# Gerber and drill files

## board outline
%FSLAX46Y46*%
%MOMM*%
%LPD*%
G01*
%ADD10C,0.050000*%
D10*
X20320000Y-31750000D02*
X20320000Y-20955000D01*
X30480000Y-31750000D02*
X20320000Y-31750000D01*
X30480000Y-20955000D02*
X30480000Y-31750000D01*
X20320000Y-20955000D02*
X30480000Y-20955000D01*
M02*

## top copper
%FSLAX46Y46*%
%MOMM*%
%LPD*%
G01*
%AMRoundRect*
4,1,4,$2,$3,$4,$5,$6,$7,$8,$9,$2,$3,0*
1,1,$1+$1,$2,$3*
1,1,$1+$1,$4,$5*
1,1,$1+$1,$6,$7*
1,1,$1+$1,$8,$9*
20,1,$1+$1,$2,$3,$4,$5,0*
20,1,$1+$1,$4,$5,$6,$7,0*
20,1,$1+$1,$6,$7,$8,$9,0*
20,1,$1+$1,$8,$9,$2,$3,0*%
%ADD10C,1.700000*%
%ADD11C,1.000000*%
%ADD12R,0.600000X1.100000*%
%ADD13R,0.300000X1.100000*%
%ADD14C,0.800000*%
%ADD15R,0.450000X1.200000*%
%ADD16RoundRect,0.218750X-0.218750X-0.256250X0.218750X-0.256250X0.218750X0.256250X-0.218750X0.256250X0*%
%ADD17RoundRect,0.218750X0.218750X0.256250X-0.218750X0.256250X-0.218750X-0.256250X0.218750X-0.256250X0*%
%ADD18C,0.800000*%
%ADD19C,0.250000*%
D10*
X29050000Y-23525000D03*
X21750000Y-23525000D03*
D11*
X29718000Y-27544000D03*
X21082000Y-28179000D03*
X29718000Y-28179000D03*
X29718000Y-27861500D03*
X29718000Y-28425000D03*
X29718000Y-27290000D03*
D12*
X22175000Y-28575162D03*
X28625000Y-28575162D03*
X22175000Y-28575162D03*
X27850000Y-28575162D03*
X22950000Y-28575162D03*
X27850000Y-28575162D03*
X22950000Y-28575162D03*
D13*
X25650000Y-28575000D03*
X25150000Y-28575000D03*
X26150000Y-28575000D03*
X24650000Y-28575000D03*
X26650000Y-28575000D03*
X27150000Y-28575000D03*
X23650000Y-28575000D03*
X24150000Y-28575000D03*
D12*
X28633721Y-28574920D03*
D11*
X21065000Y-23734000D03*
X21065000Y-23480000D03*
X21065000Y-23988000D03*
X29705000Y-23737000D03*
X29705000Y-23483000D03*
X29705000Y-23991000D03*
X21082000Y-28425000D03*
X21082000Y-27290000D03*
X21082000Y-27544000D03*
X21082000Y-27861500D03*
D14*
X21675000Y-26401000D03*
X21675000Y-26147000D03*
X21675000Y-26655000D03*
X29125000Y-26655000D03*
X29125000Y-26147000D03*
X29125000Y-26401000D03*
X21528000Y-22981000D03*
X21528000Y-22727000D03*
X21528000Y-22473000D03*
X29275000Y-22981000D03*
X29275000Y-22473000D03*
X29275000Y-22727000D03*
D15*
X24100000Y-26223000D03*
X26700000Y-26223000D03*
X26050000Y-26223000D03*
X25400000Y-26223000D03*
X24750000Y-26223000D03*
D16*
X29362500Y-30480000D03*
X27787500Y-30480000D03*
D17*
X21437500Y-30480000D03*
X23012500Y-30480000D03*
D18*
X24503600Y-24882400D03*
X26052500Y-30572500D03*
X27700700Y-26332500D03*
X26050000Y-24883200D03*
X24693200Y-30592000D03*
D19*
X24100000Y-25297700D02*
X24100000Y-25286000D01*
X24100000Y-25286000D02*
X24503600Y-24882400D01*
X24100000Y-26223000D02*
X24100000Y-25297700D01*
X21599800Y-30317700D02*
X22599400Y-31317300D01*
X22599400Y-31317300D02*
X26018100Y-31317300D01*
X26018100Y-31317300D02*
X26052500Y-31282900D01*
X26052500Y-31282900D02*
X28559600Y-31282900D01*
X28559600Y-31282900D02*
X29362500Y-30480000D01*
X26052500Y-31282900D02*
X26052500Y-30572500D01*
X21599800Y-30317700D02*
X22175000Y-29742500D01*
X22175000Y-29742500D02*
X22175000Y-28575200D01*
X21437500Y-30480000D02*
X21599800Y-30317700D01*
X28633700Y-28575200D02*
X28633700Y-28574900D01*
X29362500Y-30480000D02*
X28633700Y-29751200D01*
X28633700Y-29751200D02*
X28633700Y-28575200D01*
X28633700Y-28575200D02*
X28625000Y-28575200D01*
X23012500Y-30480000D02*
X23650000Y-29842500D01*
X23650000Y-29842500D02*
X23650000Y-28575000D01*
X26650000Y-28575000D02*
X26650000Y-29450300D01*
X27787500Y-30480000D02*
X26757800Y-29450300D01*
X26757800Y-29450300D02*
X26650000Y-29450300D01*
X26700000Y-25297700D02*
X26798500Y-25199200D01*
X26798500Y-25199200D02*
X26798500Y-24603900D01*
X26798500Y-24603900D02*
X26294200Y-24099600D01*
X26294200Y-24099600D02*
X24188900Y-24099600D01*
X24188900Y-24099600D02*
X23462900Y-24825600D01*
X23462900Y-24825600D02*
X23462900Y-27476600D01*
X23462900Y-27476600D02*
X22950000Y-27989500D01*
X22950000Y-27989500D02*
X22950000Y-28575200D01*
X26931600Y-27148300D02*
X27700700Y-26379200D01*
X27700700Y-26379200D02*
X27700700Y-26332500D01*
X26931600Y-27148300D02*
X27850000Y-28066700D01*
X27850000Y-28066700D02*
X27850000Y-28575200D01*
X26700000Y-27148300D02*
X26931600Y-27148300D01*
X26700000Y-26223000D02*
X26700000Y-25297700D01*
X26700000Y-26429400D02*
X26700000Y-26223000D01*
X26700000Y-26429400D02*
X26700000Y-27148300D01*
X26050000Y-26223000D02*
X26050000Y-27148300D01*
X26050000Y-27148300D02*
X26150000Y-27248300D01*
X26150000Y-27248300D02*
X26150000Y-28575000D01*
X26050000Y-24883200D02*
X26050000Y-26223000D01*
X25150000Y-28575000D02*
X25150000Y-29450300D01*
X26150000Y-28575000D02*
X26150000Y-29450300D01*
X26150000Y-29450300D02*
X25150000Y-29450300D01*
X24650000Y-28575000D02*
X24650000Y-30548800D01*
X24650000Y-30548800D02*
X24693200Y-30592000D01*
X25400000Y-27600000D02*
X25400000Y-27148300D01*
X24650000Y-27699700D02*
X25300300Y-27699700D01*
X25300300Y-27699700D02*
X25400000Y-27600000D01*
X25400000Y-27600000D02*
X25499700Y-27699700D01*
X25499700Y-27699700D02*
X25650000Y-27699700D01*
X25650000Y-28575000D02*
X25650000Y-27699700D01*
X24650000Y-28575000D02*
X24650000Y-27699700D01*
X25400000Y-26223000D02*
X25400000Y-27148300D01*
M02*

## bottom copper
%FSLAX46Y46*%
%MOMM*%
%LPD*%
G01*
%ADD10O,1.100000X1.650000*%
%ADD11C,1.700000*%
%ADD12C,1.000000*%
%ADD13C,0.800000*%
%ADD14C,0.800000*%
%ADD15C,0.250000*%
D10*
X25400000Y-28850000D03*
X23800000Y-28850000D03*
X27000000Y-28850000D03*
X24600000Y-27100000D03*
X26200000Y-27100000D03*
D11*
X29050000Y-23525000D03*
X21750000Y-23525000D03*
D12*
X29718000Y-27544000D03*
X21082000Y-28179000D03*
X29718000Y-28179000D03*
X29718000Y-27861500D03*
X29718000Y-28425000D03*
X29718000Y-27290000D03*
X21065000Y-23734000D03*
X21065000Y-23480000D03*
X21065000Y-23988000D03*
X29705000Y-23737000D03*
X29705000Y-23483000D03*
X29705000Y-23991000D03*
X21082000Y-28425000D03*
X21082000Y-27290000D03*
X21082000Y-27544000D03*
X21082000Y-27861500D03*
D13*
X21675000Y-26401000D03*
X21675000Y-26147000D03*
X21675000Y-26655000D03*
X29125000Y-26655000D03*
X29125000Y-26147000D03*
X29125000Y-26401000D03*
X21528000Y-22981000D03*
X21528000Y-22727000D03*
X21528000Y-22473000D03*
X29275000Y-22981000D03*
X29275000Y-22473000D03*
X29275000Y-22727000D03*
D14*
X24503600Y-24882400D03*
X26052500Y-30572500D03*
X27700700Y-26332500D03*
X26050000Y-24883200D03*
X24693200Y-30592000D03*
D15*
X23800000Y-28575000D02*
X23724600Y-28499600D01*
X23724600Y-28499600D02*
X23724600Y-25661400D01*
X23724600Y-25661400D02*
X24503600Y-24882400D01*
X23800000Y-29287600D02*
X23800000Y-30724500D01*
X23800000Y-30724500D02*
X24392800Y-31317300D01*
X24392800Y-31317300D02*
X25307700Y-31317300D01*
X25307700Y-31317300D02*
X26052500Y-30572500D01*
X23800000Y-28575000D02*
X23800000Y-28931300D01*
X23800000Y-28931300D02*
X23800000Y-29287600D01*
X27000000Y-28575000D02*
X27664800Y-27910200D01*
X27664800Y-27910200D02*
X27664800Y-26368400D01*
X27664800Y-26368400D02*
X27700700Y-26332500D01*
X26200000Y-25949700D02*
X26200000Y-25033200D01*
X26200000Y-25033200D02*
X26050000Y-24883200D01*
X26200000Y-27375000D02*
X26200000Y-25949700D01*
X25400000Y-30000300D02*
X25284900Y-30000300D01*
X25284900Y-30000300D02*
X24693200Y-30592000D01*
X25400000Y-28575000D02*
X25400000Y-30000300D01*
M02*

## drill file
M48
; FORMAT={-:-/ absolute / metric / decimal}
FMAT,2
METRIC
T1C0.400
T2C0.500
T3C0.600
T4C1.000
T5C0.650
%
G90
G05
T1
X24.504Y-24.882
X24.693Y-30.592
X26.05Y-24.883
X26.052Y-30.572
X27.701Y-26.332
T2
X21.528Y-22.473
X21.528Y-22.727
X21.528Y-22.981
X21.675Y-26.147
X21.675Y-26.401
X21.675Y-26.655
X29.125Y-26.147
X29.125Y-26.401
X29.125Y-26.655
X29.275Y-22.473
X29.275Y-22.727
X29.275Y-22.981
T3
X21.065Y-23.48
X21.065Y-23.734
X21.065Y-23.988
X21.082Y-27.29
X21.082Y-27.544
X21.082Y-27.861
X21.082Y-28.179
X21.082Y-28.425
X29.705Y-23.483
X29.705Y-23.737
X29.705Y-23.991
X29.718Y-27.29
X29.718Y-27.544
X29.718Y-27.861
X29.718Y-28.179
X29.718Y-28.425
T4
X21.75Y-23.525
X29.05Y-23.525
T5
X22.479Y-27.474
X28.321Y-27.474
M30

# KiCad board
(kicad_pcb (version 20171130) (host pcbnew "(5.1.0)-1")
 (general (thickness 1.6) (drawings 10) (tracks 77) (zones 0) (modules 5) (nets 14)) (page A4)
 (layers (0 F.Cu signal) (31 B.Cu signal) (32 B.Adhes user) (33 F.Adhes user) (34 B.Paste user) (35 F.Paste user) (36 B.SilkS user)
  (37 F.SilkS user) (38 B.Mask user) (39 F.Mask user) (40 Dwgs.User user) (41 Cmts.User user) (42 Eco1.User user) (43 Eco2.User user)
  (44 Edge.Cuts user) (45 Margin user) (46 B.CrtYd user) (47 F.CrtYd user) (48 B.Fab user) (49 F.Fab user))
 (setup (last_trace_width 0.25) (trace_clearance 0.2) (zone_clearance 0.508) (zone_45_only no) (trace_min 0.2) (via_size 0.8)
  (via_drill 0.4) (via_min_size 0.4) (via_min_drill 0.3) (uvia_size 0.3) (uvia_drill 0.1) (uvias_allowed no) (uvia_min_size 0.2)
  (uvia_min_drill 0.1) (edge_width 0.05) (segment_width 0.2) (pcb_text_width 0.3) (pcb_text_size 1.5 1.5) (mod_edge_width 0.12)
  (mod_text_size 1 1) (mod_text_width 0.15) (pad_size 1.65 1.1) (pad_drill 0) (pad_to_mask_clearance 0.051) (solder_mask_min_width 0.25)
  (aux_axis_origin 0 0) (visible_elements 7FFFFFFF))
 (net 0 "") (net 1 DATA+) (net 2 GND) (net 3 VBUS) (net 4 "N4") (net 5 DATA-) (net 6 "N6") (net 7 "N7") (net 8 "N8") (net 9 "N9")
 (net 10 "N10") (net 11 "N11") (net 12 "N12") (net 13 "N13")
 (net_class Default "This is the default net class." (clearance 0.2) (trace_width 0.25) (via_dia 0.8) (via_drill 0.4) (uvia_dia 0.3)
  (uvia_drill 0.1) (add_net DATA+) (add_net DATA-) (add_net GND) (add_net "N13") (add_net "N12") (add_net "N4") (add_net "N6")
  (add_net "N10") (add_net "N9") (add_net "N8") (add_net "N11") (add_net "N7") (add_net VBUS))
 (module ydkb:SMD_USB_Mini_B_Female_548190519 (layer F.Cu) (at 25.4 28.575 270)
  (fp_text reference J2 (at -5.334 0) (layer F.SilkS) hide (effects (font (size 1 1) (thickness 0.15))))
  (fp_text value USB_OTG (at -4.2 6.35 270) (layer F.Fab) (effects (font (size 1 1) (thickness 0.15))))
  (pad 3 smd oval (at 0 0 270) (size 1.65 1.1) (drill (offset 0.275 0)) (layers B.Cu B.Paste B.Mask) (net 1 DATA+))
  (pad 5 smd oval (at 0 1.6 270) (size 1.65 1.1) (drill (offset 0.275 0)) (layers B.Cu B.Paste B.Mask) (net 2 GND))
  (pad 1 smd oval (at 0 -1.6 270) (size 1.65 1.1) (drill (offset 0.275 0)) (layers B.Cu B.Paste B.Mask) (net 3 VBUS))
  (pad 4 smd oval (at -1.2 0.8 270) (size 1.65 1.1) (drill (offset -0.275 0)) (layers B.Cu B.Paste B.Mask) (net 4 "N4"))
  (pad 2 smd oval (at -1.2 -0.8 270) (size 1.65 1.1) (drill (offset -0.275 0)) (layers B.Cu B.Paste B.Mask) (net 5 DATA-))
  (pad 6 thru_hole circle (at -5.05 -3.65 270) (size 1.7 1.7) (drill 1) (layers *.Cu *.Mask) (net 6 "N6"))
  (pad "" thru_hole circle (at -5.05 3.65 180) (size 1.7 1.7) (drill 1) (layers *.Cu *.Mask)))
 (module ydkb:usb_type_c (layer F.Cu) (at 25.4 21.067)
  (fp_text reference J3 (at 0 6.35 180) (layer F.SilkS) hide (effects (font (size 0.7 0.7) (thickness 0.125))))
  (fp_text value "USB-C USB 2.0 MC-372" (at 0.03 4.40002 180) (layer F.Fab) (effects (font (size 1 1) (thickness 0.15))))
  (pad "" thru_hole circle (at 4.318 6.477 180) (size 1 1) (drill 0.6) (layers *.Cu *.Mask))
  (pad "" thru_hole circle (at -4.318 7.112 180) (size 1 1) (drill 0.6) (layers *.Cu *.Mask))
  (pad "" thru_hole circle (at 4.318 7.112 180) (size 1 1) (drill 0.6) (layers *.Cu *.Mask))
  (pad "" thru_hole circle (at 4.318 6.7945 180) (size 1 1) (drill 0.6) (layers *.Cu *.Mask))
  (pad "" thru_hole circle (at 4.318 7.358 180) (size 1 1) (drill 0.6) (layers *.Cu *.Mask))
  (pad S1 thru_hole circle (at 4.318 6.223 180) (size 1 1) (drill 0.6) (layers *.Cu *.Mask) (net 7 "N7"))
  (pad A1 smd rect (at -3.225 7.508162) (size 0.6 1.1) (layers F.Cu F.Paste F.Mask) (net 2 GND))
  (pad A12 smd rect (at 3.225 7.508162) (size 0.6 1.1) (layers F.Cu F.Paste F.Mask) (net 2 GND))
  (pad B12 smd rect (at -3.225 7.508162) (size 0.6 1.1) (layers F.Cu F.Paste F.Mask) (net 2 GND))
  (pad A9 smd rect (at 2.45 7.508162) (size 0.6 1.1) (layers F.Cu F.Paste F.Mask) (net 3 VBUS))
  (pad B9 smd rect (at -2.45 7.508162) (size 0.6 1.1) (layers F.Cu F.Paste F.Mask) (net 3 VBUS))
  (pad B4 smd rect (at 2.45 7.508162) (size 0.6 1.1) (layers F.Cu F.Paste F.Mask) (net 3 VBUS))
  (pad A4 smd rect (at -2.45 7.508162) (size 0.6 1.1) (layers F.Cu F.Paste F.Mask) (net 3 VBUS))
  (pad "" np_thru_hole circle (at -2.921 6.407 180) (size 0.65 0.65) (drill 0.65) (layers *.Cu *.Mask))
  (pad "" np_thru_hole circle (at 2.921 6.407 180) (size 0.65 0.65) (drill 0.65) (layers *.Cu *.Mask))
  (pad B6 smd rect (at 0.25 7.508) (size 0.3 1.1) (layers F.Cu F.Paste F.Mask) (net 1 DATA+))
  (pad B7 smd rect (at -0.25 7.508) (size 0.3 1.1) (layers F.Cu F.Paste F.Mask) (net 5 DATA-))
  (pad A7 smd rect (at 0.75 7.508) (size 0.3 1.1) (layers F.Cu F.Paste F.Mask) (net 5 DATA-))
  (pad A6 smd rect (at -0.75 7.508) (size 0.3 1.1) (layers F.Cu F.Paste F.Mask) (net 1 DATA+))
  (pad B5 smd rect (at 1.25 7.508) (size 0.3 1.1) (layers F.Cu F.Paste F.Mask) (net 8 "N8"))
  (pad A8 smd rect (at 1.75 7.508) (size 0.3 1.1) (layers F.Cu F.Paste F.Mask) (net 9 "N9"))
  (pad A5 smd rect (at -1.75 7.508) (size 0.3 1.1) (layers F.Cu F.Paste F.Mask) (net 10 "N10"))
  (pad B8 smd rect (at -1.25 7.508) (size 0.3 1.1) (layers F.Cu F.Paste F.Mask) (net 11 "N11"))
  (pad B1 smd rect (at 3.233721 7.50792) (size 0.6 1.1) (layers F.Cu F.Paste F.Mask) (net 2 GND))
  (pad "" thru_hole circle (at -4.335 2.667 180) (size 1 1) (drill 0.6) (layers *.Cu *.Mask))
  (pad "" thru_hole circle (at -4.335 2.413 180) (size 1 1) (drill 0.6) (layers *.Cu *.Mask))
  (pad "" thru_hole circle (at -4.335 2.921 180) (size 1 1) (drill 0.6) (layers *.Cu *.Mask))
  (pad "" thru_hole circle (at 4.305 2.67 180) (size 1 1) (drill 0.6) (layers *.Cu *.Mask))
  (pad "" thru_hole circle (at 4.305 2.416 180) (size 1 1) (drill 0.6) (layers *.Cu *.Mask))
  (pad "" thru_hole circle (at 4.305 2.924 180) (size 1 1) (drill 0.6) (layers *.Cu *.Mask))
  (pad "" thru_hole circle (at -4.318 7.358 180) (size 1 1) (drill 0.6) (layers *.Cu *.Mask))
  (pad "" thru_hole circle (at -4.318 6.223 180) (size 1 1) (drill 0.6) (layers *.Cu *.Mask))
  (pad "" thru_hole circle (at -4.318 6.477 180) (size 1 1) (drill 0.6) (layers *.Cu *.Mask))
  (pad "" thru_hole circle (at -4.318 6.7945 180) (size 1 1) (drill 0.6) (layers *.Cu *.Mask)))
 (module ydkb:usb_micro (layer F.Cu) (at 25.4 21.067 180)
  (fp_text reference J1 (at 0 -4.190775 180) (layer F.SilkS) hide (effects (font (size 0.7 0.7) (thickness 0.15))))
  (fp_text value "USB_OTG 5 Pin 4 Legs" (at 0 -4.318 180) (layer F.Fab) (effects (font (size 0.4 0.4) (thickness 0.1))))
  (pad "" thru_hole circle (at 3.725 -5.334 180) (size 0.8 0.8) (drill 0.5) (layers *.Cu *.Mask))
  (pad "" thru_hole circle (at 3.725 -5.08 180) (size 0.8 0.8) (drill 0.5) (layers *.Cu *.Mask))
  (pad "" thru_hole circle (at 3.725 -5.588 180) (size 0.8 0.8) (drill 0.5) (layers *.Cu *.Mask))
  (pad "" thru_hole circle (at -3.725 -5.588 180) (size 0.8 0.8) (drill 0.5) (layers *.Cu *.Mask))
  (pad "" thru_hole circle (at -3.725 -5.08 180) (size 0.8 0.8) (drill 0.5) (layers *.Cu *.Mask))
  (pad "" thru_hole circle (at -3.725 -5.334 180) (size 0.8 0.8) (drill 0.5) (layers *.Cu *.Mask))
  (pad "" thru_hole circle (at 3.872 -1.914 180) (size 0.8 0.8) (drill 0.5) (layers *.Cu *.Mask))
  (pad "" thru_hole circle (at 3.872 -1.66 180) (size 0.8 0.8) (drill 0.5) (layers *.Cu *.Mask))
  (pad "" thru_hole circle (at 3.872 -1.406 180) (size 0.8 0.8) (drill 0.5) (layers *.Cu *.Mask))
  (pad 6 thru_hole circle (at -3.875 -1.914 180) (size 0.8 0.8) (drill 0.5) (layers *.Cu *.Mask) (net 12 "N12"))
  (pad "" thru_hole circle (at -3.875 -1.406 180) (size 0.8 0.8) (drill 0.5) (layers *.Cu *.Mask))
  (pad "" thru_hole circle (at -3.875 -1.66 180) (size 0.8 0.8) (drill 0.5) (layers *.Cu *.Mask))
  (pad 5 smd rect (at 1.3 -5.156 180) (size 0.45 1.2) (layers F.Cu F.Paste F.Mask) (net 2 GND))
  (pad 1 smd rect (at -1.3 -5.156 180) (size 0.45 1.2) (layers F.Cu F.Paste F.Mask) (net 3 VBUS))
  (pad 2 smd rect (at -0.65 -5.156 180) (size 0.45 1.2) (layers F.Cu F.Paste F.Mask) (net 5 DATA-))
  (pad 3 smd rect (at 0 -5.156 180) (size 0.45 1.2) (layers F.Cu F.Paste F.Mask) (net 1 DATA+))
  (pad 4 smd rect (at 0.65 -5.156 180) (size 0.45 1.2) (layers F.Cu F.Paste F.Mask) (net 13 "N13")))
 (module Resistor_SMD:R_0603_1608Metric (layer F.Cu) (at 28.575 30.48)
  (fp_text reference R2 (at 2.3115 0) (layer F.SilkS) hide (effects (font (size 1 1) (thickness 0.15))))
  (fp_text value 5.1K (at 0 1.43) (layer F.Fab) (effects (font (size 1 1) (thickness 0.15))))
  (pad 2 smd roundrect (at 0.7875 0) (size 0.875 0.95) (layers F.Cu F.Paste F.Mask) (roundrect_rratio 0.25) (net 2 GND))
  (pad 1 smd roundrect (at -0.7875 0) (size 0.875 0.95) (layers F.Cu F.Paste F.Mask) (roundrect_rratio 0.25) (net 8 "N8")))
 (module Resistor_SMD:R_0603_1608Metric (layer F.Cu) (at 22.225 30.48 180)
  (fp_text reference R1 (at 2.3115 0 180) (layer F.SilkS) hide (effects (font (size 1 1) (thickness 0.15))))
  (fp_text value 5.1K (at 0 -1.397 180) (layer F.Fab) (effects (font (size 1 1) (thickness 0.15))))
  (pad 2 smd roundrect (at 0.7875 0 180) (size 0.875 0.95) (layers F.Cu F.Paste F.Mask) (roundrect_rratio 0.25) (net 2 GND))
  (pad 1 smd roundrect (at -0.7875 0 180) (size 0.875 0.95) (layers F.Cu F.Paste F.Mask) (roundrect_rratio 0.25) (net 10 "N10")))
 (gr_line (start 20.32 31.75) (end 20.32 20.955) (layer Edge.Cuts) (width 0.05))
 (gr_line (start 30.48 31.75) (end 20.32 31.75) (layer Edge.Cuts) (width 0.05))
 (gr_line (start 30.48 20.955) (end 30.48 31.75) (layer Edge.Cuts) (width 0.05))
 (gr_line (start 20.32 20.955) (end 30.48 20.955) (layer Edge.Cuts) (width 0.05))
 (segment (start 24.1 25.2977) (end 24.1 25.286) (width 0.25) (layer F.Cu) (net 2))
 (segment (start 24.1 25.286) (end 24.5036 24.8824) (width 0.25) (layer F.Cu) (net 2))
 (segment (start 23.8 28.575) (end 23.7246 28.4996) (width 0.25) (layer B.Cu) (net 2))
 (segment (start 23.7246 28.4996) (end 23.7246 25.6614) (width 0.25) (layer B.Cu) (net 2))
 (segment (start 23.7246 25.6614) (end 24.5036 24.8824) (width 0.25) (layer B.Cu) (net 2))
 (segment (start 24.1 26.223) (end 24.1 25.2977) (width 0.25) (layer F.Cu) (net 2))
 (segment (start 23.8 29.2876) (end 23.8 30.7245) (width 0.25) (layer B.Cu) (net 2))
 (segment (start 23.8 30.7245) (end 24.3928 31.3173) (width 0.25) (layer B.Cu) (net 2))
 (segment (start 24.3928 31.3173) (end 25.3077 31.3173) (width 0.25) (layer B.Cu) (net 2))
 (segment (start 25.3077 31.3173) (end 26.0525 30.5725) (width 0.25) (layer B.Cu) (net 2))
 (segment (start 21.5998 30.3177) (end 22.5994 31.3173) (width 0.25) (layer F.Cu) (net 2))
 (segment (start 22.5994 31.3173) (end 26.0181 31.3173) (width 0.25) (layer F.Cu) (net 2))
 (segment (start 26.0181 31.3173) (end 26.0525 31.2829) (width 0.25) (layer F.Cu) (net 2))
 (segment (start 26.0525 31.2829) (end 28.5596 31.2829) (width 0.25) (layer F.Cu) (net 2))
 (segment (start 28.5596 31.2829) (end 29.3625 30.48) (width 0.25) (layer F.Cu) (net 2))
 (segment (start 26.0525 31.2829) (end 26.0525 30.5725) (width 0.25) (layer F.Cu) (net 2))
 (segment (start 23.8 28.575) (end 23.8 28.9313) (width 0.25) (layer B.Cu) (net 2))
 (segment (start 23.8 28.9313) (end 23.8 29.2876) (width 0.25) (layer B.Cu) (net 2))
 (segment (start 21.5998 30.3177) (end 22.175 29.7425) (width 0.25) (layer F.Cu) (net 2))
 (segment (start 22.175 29.7425) (end 22.175 28.5752) (width 0.25) (layer F.Cu) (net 2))
 (segment (start 21.4375 30.48) (end 21.5998 30.3177) (width 0.25) (layer F.Cu) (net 2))
 (segment (start 28.6337 28.5752) (end 28.6337 28.5749) (width 0.25) (layer F.Cu) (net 2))
 (segment (start 29.3625 30.48) (end 28.6337 29.7512) (width 0.25) (layer F.Cu) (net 2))
 (segment (start 28.6337 29.7512) (end 28.6337 28.5752) (width 0.25) (layer F.Cu) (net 2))
 (segment (start 28.6337 28.5752) (end 28.625 28.5752) (width 0.25) (layer F.Cu) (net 2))
 (via (at 24.5036 24.8824) (size 0.8) (layers F.Cu B.Cu) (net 2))
 (via (at 26.0525 30.5725) (size 0.8) (layers F.Cu B.Cu) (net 2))
 (segment (start 23.0125 30.48) (end 23.65 29.8425) (width 0.25) (layer F.Cu) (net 10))
 (segment (start 23.65 29.8425) (end 23.65 28.575) (width 0.25) (layer F.Cu) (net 10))
 (segment (start 26.65 28.575) (end 26.65 29.4503) (width 0.25) (layer F.Cu) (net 8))
 (segment (start 27.7875 30.48) (end 26.7578 29.4503) (width 0.25) (layer F.Cu) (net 8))
 (segment (start 26.7578 29.4503) (end 26.65 29.4503) (width 0.25) (layer F.Cu) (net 8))
 (segment (start 26.7 25.2977) (end 26.7985 25.1992) (width 0.25) (layer F.Cu) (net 3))
 (segment (start 26.7985 25.1992) (end 26.7985 24.6039) (width 0.25) (layer F.Cu) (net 3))
 (segment (start 26.7985 24.6039) (end 26.2942 24.0996) (width 0.25) (layer F.Cu) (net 3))
 (segment (start 26.2942 24.0996) (end 24.1889 24.0996) (width 0.25) (layer F.Cu) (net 3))
 (segment (start 24.1889 24.0996) (end 23.4629 24.8256) (width 0.25) (layer F.Cu) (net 3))
 (segment (start 23.4629 24.8256) (end 23.4629 27.4766) (width 0.25) (layer F.Cu) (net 3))
 (segment (start 23.4629 27.4766) (end 22.95 27.9895) (width 0.25) (layer F.Cu) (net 3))
 (segment (start 22.95 27.9895) (end 22.95 28.5752) (width 0.25) (layer F.Cu) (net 3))
 (segment (start 26.9316 27.1483) (end 27.7007 26.3792) (width 0.25) (layer F.Cu) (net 3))
 (segment (start 27.7007 26.3792) (end 27.7007 26.3325) (width 0.25) (layer F.Cu) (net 3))
 (segment (start 27 28.575) (end 27.6648 27.9102) (width 0.25) (layer B.Cu) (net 3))
 (segment (start 27.6648 27.9102) (end 27.6648 26.3684) (width 0.25) (layer B.Cu) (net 3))
 (segment (start 27.6648 26.3684) (end 27.7007 26.3325) (width 0.25) (layer B.Cu) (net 3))
 (segment (start 26.9316 27.1483) (end 27.85 28.0667) (width 0.25) (layer F.Cu) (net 3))
 (segment (start 27.85 28.0667) (end 27.85 28.5752) (width 0.25) (layer F.Cu) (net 3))
 (segment (start 26.7 27.1483) (end 26.9316 27.1483) (width 0.25) (layer F.Cu) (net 3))
 (segment (start 26.7 26.223) (end 26.7 25.2977) (width 0.25) (layer F.Cu) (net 3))
 (segment (start 26.7 26.4294) (end 26.7 26.223) (width 0.25) (layer F.Cu) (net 3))
 (segment (start 26.7 26.4294) (end 26.7 27.1483) (width 0.25) (layer F.Cu) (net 3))
 (via (at 27.7007 26.3325) (size 0.8) (layers F.Cu B.Cu) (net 3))
 (segment (start 26.05 26.223) (end 26.05 27.1483) (width 0.25) (layer F.Cu) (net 5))
 (segment (start 26.05 27.1483) (end 26.15 27.2483) (width 0.25) (layer F.Cu) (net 5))
 (segment (start 26.15 27.2483) (end 26.15 28.575) (width 0.25) (layer F.Cu) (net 5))
 (segment (start 26.05 24.8832) (end 26.05 26.223) (width 0.25) (layer F.Cu) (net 5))
 (segment (start 26.2 25.9497) (end 26.2 25.0332) (width 0.25) (layer B.Cu) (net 5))
 (segment (start 26.2 25.0332) (end 26.05 24.8832) (width 0.25) (layer B.Cu) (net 5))
 (segment (start 26.2 27.375) (end 26.2 25.9497) (width 0.25) (layer B.Cu) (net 5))
 (segment (start 25.15 28.575) (end 25.15 29.4503) (width 0.25) (layer F.Cu) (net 5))
 (segment (start 26.15 28.575) (end 26.15 29.4503) (width 0.25) (layer F.Cu) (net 5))
 (segment (start 26.15 29.4503) (end 25.15 29.4503) (width 0.25) (layer F.Cu) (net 5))
 (via (at 26.05 24.8832) (size 0.8) (layers F.Cu B.Cu) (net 5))
 (segment (start 24.65 28.575) (end 24.65 30.5488) (width 0.25) (layer F.Cu) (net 1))
 (segment (start 24.65 30.5488) (end 24.6932 30.592) (width 0.25) (layer F.Cu) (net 1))
 (segment (start 25.4 30.0003) (end 25.2849 30.0003) (width 0.25) (layer B.Cu) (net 1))
 (segment (start 25.2849 30.0003) (end 24.6932 30.592) (width 0.25) (layer B.Cu) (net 1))
 (segment (start 25.4 27.6) (end 25.4 27.1483) (width 0.25) (layer F.Cu) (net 1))
 (segment (start 24.65 27.6997) (end 25.3003 27.6997) (width 0.25) (layer F.Cu) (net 1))
 (segment (start 25.3003 27.6997) (end 25.4 27.6) (width 0.25) (layer F.Cu) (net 1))
 (segment (start 25.4 27.6) (end 25.4997 27.6997) (width 0.25) (layer F.Cu) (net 1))
 (segment (start 25.4997 27.6997) (end 25.65 27.6997) (width 0.25) (layer F.Cu) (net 1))
 (segment (start 25.65 28.575) (end 25.65 27.6997) (width 0.25) (layer F.Cu) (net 1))
 (segment (start 24.65 28.575) (end 24.65 27.6997) (width 0.25) (layer F.Cu) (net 1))
 (segment (start 25.4 26.223) (end 25.4 27.1483) (width 0.25) (layer F.Cu) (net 1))
 (segment (start 25.4 28.575) (end 25.4 30.0003) (width 0.25) (layer B.Cu) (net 1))
 (via (at 24.6932 30.592) (size 0.8) (layers F.Cu B.Cu) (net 1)))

